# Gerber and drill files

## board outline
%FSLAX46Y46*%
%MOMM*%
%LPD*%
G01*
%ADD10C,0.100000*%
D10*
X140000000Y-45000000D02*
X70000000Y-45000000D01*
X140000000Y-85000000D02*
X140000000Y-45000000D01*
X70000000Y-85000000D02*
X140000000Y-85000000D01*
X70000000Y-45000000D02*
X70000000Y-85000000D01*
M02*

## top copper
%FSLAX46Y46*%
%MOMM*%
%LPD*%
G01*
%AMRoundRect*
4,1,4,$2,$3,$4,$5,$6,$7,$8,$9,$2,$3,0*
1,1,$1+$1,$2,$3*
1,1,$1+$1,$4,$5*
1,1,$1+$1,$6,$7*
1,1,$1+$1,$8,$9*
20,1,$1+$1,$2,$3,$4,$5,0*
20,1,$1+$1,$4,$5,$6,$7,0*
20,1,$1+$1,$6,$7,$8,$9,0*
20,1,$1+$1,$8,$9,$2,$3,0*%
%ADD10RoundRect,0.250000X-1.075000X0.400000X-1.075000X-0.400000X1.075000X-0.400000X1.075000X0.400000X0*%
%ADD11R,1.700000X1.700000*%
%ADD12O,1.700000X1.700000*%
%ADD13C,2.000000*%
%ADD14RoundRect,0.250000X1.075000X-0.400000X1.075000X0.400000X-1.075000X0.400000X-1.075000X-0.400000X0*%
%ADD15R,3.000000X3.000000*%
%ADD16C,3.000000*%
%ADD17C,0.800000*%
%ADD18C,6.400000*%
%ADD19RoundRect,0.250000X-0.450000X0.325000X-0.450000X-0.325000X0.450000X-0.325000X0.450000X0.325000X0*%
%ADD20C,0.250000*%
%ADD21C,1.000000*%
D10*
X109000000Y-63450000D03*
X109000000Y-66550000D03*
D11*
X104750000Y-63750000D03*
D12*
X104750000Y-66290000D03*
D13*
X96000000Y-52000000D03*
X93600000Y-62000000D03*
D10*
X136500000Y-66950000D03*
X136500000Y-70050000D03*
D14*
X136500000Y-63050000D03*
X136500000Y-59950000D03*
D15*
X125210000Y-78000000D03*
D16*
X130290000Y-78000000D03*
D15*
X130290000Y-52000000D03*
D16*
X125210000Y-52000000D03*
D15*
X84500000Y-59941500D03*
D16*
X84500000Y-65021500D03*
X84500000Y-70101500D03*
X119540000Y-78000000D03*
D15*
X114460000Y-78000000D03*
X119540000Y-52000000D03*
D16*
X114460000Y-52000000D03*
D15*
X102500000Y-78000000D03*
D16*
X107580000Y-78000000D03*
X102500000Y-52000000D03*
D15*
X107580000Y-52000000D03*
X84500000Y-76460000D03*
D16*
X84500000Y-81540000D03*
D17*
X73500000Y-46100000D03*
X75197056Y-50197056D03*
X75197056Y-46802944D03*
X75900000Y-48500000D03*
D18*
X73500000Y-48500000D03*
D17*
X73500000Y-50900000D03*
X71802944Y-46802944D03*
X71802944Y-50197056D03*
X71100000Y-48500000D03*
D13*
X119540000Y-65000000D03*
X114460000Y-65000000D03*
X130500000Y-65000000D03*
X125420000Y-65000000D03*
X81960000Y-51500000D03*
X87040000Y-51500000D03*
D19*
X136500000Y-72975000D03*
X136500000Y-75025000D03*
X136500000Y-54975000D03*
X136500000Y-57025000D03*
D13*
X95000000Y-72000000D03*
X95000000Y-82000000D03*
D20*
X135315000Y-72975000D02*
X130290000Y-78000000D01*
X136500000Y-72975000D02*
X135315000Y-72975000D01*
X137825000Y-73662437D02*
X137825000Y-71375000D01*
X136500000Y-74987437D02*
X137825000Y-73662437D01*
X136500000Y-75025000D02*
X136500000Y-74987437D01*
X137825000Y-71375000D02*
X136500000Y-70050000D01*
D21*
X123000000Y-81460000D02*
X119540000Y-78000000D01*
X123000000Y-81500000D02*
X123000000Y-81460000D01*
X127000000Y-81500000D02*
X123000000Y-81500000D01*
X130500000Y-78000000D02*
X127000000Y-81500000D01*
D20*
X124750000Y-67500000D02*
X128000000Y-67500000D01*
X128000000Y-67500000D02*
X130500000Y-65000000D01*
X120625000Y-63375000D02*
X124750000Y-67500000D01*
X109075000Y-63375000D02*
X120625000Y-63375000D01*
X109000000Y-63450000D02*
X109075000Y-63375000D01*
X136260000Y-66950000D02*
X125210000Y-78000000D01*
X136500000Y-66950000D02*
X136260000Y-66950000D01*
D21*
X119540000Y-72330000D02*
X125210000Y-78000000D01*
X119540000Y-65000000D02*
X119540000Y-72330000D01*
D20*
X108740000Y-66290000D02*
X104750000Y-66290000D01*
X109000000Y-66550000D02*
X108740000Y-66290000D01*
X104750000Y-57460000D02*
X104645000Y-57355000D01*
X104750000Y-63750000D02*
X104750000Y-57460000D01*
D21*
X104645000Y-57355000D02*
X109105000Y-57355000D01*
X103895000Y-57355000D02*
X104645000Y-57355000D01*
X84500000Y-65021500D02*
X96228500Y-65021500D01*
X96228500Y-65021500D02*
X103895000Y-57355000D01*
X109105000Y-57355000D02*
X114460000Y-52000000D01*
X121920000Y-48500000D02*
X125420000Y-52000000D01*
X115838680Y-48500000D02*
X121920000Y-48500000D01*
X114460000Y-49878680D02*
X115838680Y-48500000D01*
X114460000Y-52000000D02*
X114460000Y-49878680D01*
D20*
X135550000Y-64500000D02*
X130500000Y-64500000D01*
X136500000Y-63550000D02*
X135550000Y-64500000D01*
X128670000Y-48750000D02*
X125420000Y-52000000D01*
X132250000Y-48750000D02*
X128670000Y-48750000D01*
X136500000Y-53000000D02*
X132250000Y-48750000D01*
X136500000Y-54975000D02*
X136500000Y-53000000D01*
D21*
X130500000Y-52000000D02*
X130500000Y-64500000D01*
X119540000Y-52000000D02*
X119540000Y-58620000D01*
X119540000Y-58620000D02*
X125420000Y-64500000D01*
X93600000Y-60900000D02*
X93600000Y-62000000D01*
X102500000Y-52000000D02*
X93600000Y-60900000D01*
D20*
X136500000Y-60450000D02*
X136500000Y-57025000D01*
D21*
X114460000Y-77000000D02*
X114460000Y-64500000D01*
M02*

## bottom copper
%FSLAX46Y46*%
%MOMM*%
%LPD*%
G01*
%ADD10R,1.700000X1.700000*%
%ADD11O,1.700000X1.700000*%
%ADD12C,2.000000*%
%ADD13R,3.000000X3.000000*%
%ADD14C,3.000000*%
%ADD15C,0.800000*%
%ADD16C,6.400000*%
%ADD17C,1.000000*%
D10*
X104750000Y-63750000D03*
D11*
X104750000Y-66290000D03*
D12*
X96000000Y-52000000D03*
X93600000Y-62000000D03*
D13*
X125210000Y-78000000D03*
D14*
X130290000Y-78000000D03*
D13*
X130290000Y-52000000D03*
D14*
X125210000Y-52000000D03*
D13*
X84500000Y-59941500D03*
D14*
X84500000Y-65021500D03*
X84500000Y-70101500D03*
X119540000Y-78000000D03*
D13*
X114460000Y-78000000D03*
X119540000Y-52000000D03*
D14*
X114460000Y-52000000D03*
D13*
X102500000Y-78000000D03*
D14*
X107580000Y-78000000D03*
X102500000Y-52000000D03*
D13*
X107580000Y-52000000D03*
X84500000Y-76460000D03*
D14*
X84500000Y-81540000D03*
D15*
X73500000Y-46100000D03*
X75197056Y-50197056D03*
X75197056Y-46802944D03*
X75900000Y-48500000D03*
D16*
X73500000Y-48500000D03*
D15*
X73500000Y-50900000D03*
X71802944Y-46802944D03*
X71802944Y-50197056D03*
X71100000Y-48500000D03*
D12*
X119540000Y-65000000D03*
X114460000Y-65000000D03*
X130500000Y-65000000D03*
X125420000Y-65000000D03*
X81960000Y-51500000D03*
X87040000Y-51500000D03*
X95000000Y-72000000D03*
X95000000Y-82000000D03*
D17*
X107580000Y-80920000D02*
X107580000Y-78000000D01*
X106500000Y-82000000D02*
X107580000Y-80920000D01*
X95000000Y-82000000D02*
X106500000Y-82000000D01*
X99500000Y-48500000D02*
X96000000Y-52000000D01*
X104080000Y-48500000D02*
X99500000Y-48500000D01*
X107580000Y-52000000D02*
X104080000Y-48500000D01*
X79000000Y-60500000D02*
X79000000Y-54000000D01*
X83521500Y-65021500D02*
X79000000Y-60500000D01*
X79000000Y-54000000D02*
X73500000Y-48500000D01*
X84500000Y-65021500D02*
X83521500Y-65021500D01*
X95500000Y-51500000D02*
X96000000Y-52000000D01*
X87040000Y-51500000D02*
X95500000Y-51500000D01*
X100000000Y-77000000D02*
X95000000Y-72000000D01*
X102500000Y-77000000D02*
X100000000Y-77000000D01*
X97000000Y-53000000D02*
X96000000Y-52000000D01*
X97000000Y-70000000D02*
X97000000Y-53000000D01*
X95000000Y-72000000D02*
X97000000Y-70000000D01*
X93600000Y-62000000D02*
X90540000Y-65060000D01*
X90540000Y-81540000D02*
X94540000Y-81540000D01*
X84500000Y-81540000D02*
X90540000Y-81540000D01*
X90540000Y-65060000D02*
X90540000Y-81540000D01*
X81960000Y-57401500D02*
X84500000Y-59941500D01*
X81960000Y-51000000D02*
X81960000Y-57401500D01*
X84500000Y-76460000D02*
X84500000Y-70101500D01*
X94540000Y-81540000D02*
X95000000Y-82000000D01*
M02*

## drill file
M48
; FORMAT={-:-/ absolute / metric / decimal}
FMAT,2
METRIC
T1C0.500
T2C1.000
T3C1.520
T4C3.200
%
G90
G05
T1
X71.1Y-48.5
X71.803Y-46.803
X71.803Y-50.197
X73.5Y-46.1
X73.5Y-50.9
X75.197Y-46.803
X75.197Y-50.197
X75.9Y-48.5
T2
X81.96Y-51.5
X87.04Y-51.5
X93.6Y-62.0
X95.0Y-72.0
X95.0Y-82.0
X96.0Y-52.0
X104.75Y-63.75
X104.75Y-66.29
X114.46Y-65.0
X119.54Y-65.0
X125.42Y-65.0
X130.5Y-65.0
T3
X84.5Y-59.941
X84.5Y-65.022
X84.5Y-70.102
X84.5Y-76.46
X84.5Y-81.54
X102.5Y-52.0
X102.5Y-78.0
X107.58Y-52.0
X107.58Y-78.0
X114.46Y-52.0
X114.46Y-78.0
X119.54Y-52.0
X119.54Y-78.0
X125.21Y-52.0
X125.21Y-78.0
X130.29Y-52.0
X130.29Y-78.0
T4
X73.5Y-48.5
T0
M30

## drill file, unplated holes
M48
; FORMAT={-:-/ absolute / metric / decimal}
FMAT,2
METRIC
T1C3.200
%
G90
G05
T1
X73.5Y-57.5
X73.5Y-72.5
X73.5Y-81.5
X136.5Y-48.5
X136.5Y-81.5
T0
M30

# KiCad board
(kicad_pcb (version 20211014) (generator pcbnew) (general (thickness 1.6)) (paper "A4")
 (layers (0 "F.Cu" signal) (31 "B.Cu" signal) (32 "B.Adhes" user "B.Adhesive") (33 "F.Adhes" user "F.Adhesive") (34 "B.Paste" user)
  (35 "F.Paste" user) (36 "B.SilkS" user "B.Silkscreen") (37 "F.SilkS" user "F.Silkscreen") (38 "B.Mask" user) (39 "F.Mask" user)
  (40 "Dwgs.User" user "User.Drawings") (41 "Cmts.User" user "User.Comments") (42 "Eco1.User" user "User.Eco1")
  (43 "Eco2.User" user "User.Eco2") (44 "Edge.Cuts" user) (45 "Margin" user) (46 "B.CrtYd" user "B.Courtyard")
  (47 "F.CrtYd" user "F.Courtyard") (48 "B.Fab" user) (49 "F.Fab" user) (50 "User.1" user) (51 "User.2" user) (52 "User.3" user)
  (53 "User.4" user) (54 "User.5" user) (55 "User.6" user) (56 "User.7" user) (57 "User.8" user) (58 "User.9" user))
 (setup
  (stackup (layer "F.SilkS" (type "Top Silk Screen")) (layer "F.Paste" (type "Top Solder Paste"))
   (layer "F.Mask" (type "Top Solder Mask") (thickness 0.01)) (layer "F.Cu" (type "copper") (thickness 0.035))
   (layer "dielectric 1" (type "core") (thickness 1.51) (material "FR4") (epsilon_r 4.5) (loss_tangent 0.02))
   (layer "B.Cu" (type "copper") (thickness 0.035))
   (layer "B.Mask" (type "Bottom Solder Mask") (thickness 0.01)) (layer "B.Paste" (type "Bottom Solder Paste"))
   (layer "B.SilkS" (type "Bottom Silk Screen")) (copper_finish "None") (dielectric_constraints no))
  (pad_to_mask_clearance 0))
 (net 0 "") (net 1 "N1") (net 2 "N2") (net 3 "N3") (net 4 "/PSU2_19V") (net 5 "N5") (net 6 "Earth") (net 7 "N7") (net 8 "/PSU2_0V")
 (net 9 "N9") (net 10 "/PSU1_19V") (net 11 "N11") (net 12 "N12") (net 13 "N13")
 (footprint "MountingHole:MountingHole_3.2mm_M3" (layer "F.Cu") (at 73.5 57.5)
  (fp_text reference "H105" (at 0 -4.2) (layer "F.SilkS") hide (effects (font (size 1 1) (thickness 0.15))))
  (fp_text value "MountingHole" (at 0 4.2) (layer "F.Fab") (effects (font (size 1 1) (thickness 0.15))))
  (pad "" np_thru_hole circle (at 0 0) (size 3.2 3.2) (drill 3.2) (layers *.Cu *.Mask)))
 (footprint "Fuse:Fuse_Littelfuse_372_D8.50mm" (layer "F.Cu") (at 81.96 51.5)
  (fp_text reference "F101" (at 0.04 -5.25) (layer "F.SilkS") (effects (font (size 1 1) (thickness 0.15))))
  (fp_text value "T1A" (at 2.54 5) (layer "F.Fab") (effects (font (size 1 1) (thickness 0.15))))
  (pad "1" thru_hole circle (at 0 0) (size 2 2) (drill 1) (layers *.Cu *.Mask) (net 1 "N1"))
  (pad "2" thru_hole circle (at 5.08 0) (size 2 2) (drill 1) (layers *.Cu *.Mask) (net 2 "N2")))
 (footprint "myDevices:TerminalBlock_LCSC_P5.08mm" (layer "F.Cu") (at 102.5 78)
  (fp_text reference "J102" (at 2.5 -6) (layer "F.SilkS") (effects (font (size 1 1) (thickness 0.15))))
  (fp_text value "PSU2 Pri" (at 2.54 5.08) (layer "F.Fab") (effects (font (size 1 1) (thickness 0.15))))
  (pad "1" thru_hole rect locked (at 0 0) (size 3 3) (drill 1.52) (layers *.Cu *.Mask) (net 2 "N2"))
  (pad "2" thru_hole circle locked (at 5.08 0) (size 3 3) (drill 1.52) (layers *.Cu *.Mask) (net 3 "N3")))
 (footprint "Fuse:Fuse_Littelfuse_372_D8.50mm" (layer "F.Cu") (at 119.54 65 180)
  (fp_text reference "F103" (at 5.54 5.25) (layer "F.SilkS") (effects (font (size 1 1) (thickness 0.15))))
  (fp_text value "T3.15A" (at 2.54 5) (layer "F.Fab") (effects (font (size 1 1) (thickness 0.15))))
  (pad "1" thru_hole circle (at 0 0 180) (size 2 2) (drill 1) (layers *.Cu *.Mask) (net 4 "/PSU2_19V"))
  (pad "2" thru_hole circle (at 5.08 0 180) (size 2 2) (drill 1) (layers *.Cu *.Mask) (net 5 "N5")))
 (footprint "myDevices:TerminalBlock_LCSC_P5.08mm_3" (layer "F.Cu") (at 84.5 59.9415 -90)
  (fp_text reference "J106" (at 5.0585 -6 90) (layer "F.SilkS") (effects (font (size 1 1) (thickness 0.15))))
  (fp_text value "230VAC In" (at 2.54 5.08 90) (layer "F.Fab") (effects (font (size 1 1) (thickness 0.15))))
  (pad "1" thru_hole rect locked (at 0 0 270) (size 3 3) (drill 1.52) (layers *.Cu *.Mask) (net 1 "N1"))
  (pad "2" thru_hole circle locked (at 5.08 0 270) (size 3 3) (drill 1.52) (layers *.Cu *.Mask) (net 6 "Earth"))
  (pad "3" thru_hole circle locked (at 10.16 0 270) (size 3 3) (drill 1.52) (layers *.Cu *.Mask) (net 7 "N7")))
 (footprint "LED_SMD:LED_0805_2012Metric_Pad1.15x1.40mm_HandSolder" (layer "F.Cu") (at 136.5 74 -90)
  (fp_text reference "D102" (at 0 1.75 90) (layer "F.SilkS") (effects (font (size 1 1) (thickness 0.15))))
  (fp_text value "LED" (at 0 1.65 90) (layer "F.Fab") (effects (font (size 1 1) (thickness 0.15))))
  (pad "1" smd roundrect (at -1.025 0 270) (size 1.15 1.4) (layers "F.Cu" "F.Paste" "F.Mask") (roundrect_rratio 0.2173913043)
   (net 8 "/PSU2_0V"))
  (pad "2" smd roundrect (at 1.025 0 270) (size 1.15 1.4) (layers "F.Cu" "F.Paste" "F.Mask") (roundrect_rratio 0.2173913043) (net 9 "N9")))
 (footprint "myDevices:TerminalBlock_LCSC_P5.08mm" (layer "F.Cu") (at 130.29 52 180)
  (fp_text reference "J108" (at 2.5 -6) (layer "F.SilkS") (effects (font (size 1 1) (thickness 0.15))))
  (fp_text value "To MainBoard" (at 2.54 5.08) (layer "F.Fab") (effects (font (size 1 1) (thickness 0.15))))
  (pad "1" thru_hole rect locked (at 0 0 180) (size 3 3) (drill 1.52) (layers *.Cu *.Mask) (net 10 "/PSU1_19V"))
  (pad "2" thru_hole circle locked (at 5.08 0 180) (size 3 3) (drill 1.52) (layers *.Cu *.Mask) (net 6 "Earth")))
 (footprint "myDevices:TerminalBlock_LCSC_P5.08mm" (layer "F.Cu") (at 84.5 76.46 -90)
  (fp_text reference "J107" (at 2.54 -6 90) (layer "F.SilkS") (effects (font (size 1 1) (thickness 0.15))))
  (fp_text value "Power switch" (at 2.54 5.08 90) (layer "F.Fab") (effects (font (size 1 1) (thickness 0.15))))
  (pad "1" thru_hole rect locked (at 0 0 270) (size 3 3) (drill 1.52) (layers *.Cu *.Mask) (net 7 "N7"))
  (pad "2" thru_hole circle locked (at 5.08 0 270) (size 3 3) (drill 1.52) (layers *.Cu *.Mask) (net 3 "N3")))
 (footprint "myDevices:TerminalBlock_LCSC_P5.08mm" (layer "F.Cu") (at 119.54 52 180)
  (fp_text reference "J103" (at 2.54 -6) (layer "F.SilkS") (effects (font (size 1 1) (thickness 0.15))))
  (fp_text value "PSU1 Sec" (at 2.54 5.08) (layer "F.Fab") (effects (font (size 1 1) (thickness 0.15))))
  (pad "1" thru_hole rect locked (at 0 0 180) (size 3 3) (drill 1.52) (layers *.Cu *.Mask) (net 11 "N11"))
  (pad "2" thru_hole circle locked (at 5.08 0 180) (size 3 3) (drill 1.52) (layers *.Cu *.Mask) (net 6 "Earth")))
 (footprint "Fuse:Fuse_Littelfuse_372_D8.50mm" (layer "F.Cu") (at 130.5 65 180)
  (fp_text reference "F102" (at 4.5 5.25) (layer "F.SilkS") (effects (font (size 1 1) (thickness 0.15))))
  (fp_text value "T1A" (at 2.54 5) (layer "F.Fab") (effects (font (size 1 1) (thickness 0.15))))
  (pad "1" thru_hole circle (at 0 0 180) (size 2 2) (drill 1) (layers *.Cu *.Mask) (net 10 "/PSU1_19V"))
  (pad "2" thru_hole circle (at 5.08 0 180) (size 2 2) (drill 1) (layers *.Cu *.Mask) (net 11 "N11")))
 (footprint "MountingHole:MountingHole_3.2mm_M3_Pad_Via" (layer "F.Cu") (at 73.5 48.5)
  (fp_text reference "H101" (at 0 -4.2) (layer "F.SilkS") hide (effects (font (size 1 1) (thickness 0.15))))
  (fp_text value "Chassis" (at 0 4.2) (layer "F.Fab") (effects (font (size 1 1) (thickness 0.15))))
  (pad "1" thru_hole circle (at 0 2.4) (size 0.8 0.8) (drill 0.5) (layers *.Cu *.Mask) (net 6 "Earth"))
  (pad "1" thru_hole circle (at 0 0) (size 6.4 6.4) (drill 3.2) (layers *.Cu *.Mask) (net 6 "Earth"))
  (pad "1" thru_hole circle (at -1.697056 1.697056) (size 0.8 0.8) (drill 0.5) (layers *.Cu *.Mask) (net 6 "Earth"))
  (pad "1" thru_hole circle (at 0 -2.4) (size 0.8 0.8) (drill 0.5) (layers *.Cu *.Mask) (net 6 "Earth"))
  (pad "1" thru_hole circle (at 1.697056 1.697056) (size 0.8 0.8) (drill 0.5) (layers *.Cu *.Mask) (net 6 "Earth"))
  (pad "1" thru_hole circle (at 1.697056 -1.697056) (size 0.8 0.8) (drill 0.5) (layers *.Cu *.Mask) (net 6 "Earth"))
  (pad "1" thru_hole circle (at 2.4 0) (size 0.8 0.8) (drill 0.5) (layers *.Cu *.Mask) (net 6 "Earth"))
  (pad "1" thru_hole circle (at -1.697056 -1.697056) (size 0.8 0.8) (drill 0.5) (layers *.Cu *.Mask) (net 6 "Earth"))
  (pad "1" thru_hole circle (at -2.4 0) (size 0.8 0.8) (drill 0.5) (layers *.Cu *.Mask) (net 6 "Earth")))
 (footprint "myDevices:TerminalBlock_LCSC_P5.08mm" (layer "F.Cu") (at 125.21 78)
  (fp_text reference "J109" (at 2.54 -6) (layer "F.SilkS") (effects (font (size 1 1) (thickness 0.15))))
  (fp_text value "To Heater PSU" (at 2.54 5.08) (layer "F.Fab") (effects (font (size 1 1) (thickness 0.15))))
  (pad "1" thru_hole rect locked (at 0 0) (size 3 3) (drill 1.52) (layers *.Cu *.Mask) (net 4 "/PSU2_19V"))
  (pad "2" thru_hole circle locked (at 5.08 0) (size 3 3) (drill 1.52) (layers *.Cu *.Mask) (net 8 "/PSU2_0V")))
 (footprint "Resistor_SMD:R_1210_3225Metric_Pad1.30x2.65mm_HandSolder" (layer "F.Cu") (at 136.5 68.5 -90)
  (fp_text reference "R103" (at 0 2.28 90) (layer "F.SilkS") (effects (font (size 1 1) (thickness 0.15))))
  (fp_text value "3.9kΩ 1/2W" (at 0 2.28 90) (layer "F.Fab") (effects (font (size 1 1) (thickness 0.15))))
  (pad "1" smd roundrect (at -1.55 0 270) (size 1.3 2.65) (layers "F.Cu" "F.Paste" "F.Mask") (roundrect_rratio 0.1923076923)
   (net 4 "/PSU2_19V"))
  (pad "2" smd roundrect (at 1.55 0 270) (size 1.3 2.65) (layers "F.Cu" "F.Paste" "F.Mask") (roundrect_rratio 0.1923076923) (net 9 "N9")))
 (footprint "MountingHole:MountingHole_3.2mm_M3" (layer "F.Cu") (at 73.5 81.5)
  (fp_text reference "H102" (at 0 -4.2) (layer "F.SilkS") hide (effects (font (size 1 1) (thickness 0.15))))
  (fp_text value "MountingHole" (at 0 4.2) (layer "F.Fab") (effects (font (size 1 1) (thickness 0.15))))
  (pad "" np_thru_hole circle (at 0 0) (size 3.2 3.2) (drill 3.2) (layers *.Cu *.Mask)))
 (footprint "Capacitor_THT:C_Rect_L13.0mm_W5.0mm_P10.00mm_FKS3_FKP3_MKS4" (layer "F.Cu") (at 95 72 -90)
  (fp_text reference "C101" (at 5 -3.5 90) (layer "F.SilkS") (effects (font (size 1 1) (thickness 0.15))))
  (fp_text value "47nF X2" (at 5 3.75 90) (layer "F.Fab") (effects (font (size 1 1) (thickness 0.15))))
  (pad "1" thru_hole circle (at 0 0 270) (size 2 2) (drill 1) (layers *.Cu *.Mask) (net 2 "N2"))
  (pad "2" thru_hole circle (at 10 0 270) (size 2 2) (drill 1) (layers *.Cu *.Mask) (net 3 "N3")))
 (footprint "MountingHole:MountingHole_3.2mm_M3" (layer "F.Cu") (at 136.5 81.5)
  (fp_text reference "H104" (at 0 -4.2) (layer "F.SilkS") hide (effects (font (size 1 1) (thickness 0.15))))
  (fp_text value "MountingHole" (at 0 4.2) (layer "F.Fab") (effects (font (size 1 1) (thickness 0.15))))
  (pad "" np_thru_hole circle (at 0 0) (size 3.2 3.2) (drill 3.2) (layers *.Cu *.Mask)))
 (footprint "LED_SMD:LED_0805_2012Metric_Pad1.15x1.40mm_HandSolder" (layer "F.Cu") (at 136.5 56 -90)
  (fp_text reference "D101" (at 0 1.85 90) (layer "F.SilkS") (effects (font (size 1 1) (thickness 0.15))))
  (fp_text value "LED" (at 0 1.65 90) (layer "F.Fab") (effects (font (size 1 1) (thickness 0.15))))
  (pad "1" smd roundrect (at -1.025 0 270) (size 1.15 1.4) (layers "F.Cu" "F.Paste" "F.Mask") (roundrect_rratio 0.2173913043)
   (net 6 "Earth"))
  (pad "2" smd roundrect (at 1.025 0 270) (size 1.15 1.4) (layers "F.Cu" "F.Paste" "F.Mask") (roundrect_rratio 0.2173913043) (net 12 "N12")))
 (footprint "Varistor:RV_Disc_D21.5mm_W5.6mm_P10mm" (layer "F.Cu") (at 96 52 -90)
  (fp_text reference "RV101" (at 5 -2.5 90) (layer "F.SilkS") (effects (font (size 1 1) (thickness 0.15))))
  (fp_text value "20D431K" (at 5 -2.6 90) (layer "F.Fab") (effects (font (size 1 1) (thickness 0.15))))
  (pad "1" thru_hole circle (at 0 0 270) (size 2 2) (drill 1) (layers *.Cu *.Mask) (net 2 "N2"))
  (pad "2" thru_hole circle (at 10 2.4 270) (size 2 2) (drill 1) (layers *.Cu *.Mask) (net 3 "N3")))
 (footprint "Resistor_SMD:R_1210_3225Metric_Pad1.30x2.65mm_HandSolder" (layer "F.Cu") (at 136.5 61.5 90)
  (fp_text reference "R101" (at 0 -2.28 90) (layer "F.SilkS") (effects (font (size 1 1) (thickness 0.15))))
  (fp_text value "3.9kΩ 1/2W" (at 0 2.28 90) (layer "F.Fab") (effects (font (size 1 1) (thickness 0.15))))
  (pad "1" smd roundrect (at -1.55 0 90) (size 1.3 2.65) (layers "F.Cu" "F.Paste" "F.Mask") (roundrect_rratio 0.1923076923)
   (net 10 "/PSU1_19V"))
  (pad "2" smd roundrect (at 1.55 0 90) (size 1.3 2.65) (layers "F.Cu" "F.Paste" "F.Mask") (roundrect_rratio 0.1923076923) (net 12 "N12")))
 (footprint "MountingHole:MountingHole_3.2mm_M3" (layer "F.Cu") (at 136.5 48.5)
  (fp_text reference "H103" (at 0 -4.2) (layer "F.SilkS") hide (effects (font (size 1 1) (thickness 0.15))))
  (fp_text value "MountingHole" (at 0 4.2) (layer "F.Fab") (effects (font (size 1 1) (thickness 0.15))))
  (pad "" np_thru_hole circle (at 0 0) (size 3.2 3.2) (drill 3.2) (layers *.Cu *.Mask)))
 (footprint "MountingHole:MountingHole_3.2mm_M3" (layer "F.Cu") (at 73.5 72.5)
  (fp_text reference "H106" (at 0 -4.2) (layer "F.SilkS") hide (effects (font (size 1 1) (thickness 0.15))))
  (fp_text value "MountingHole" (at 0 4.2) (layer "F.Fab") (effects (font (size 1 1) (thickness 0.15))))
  (pad "" np_thru_hole circle (at 0 0) (size 3.2 3.2) (drill 3.2) (layers *.Cu *.Mask)))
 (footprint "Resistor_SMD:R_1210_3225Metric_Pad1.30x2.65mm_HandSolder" (layer "F.Cu") (at 109 65 -90)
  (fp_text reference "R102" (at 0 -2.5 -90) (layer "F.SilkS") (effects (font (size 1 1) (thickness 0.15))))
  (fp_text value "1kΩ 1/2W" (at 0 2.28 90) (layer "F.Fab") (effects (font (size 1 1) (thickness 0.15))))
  (pad "1" smd roundrect (at -1.55 0 270) (size 1.3 2.65) (layers "F.Cu" "F.Paste" "F.Mask") (roundrect_rratio 0.1923076923)
   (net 10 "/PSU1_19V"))
  (pad "2" smd roundrect (at 1.55 0 270) (size 1.3 2.65) (layers "F.Cu" "F.Paste" "F.Mask") (roundrect_rratio 0.1923076923) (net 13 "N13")))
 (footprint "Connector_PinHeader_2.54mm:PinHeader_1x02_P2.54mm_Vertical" (layer "F.Cu") (at 104.75 63.75)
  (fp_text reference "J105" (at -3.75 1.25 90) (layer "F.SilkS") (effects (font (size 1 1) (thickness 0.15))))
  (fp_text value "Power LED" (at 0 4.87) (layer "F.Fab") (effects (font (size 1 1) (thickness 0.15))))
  (pad "1" thru_hole rect (at 0 0) (size 1.7 1.7) (drill 1) (layers *.Cu *.Mask) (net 6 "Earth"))
  (pad "2" thru_hole oval (at 0 2.54) (size 1.7 1.7) (drill 1) (layers *.Cu *.Mask) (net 13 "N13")))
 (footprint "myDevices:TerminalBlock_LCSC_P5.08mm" (layer "F.Cu") (at 114.46 78)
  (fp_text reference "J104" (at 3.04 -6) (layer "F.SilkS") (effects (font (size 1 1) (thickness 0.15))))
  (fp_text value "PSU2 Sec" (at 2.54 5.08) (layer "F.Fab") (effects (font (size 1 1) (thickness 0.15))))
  (pad "1" thru_hole rect locked (at 0 0) (size 3 3) (drill 1.52) (layers *.Cu *.Mask) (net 5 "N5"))
  (pad "2" thru_hole circle locked (at 5.08 0) (size 3 3) (drill 1.52) (layers *.Cu *.Mask) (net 8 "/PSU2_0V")))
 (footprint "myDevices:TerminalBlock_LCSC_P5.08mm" (layer "F.Cu") (at 107.58 52 180)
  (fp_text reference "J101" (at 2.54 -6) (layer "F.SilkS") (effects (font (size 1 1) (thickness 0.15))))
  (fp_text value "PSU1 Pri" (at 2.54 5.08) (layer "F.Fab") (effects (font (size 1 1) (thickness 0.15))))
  (pad "1" thru_hole rect locked (at 0 0 180) (size 3 3) (drill 1.52) (layers *.Cu *.Mask) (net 2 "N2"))
  (pad "2" thru_hole circle locked (at 5.08 0 180) (size 3 3) (drill 1.52) (layers *.Cu *.Mask) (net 3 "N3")))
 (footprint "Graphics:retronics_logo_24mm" (layer "B.Cu") (at 122.497465 62.25 180)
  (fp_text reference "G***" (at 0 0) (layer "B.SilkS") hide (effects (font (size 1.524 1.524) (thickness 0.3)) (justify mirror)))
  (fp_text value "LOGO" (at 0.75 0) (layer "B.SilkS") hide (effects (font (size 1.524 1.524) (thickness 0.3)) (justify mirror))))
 (gr_line (start 140 85) (end 140 45) (layer "Edge.Cuts") (width 0.1))
 (gr_line (start 140 45) (end 70 45) (layer "Edge.Cuts") (width 0.1))
 (gr_line (start 70 45) (end 70 85) (layer "Edge.Cuts") (width 0.1))
 (gr_line (start 70 85) (end 140 85) (layer "Edge.Cuts") (width 0.1))
 (segment (start 97 70) (end 97 53) (width 1) (layer "B.Cu") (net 2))
 (segment (start 102.5 77) (end 100 77) (width 1) (layer "B.Cu") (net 2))
 (segment (start 97 53) (end 96 52) (width 1) (layer "B.Cu") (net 2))
 (segment (start 104.08 48.5) (end 99.5 48.5) (width 1) (layer "B.Cu") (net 2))
 (segment (start 87.04 51.5) (end 95.5 51.5) (width 1) (layer "B.Cu") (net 2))
 (segment (start 107.58 52) (end 104.08 48.5) (width 1) (layer "B.Cu") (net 2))
 (segment (start 99.5 48.5) (end 96 52) (width 1) (layer "B.Cu") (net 2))
 (segment (start 95.5 51.5) (end 96 52) (width 1) (layer "B.Cu") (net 2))
 (segment (start 100 77) (end 95 72) (width 1) (layer "B.Cu") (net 2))
 (segment (start 95 72) (end 97 70) (width 1) (layer "B.Cu") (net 2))
 (segment (start 93.6 60.9) (end 93.6 62) (width 1) (layer "F.Cu") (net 3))
 (segment (start 102.5 52) (end 93.6 60.9) (width 1) (layer "F.Cu") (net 3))
 (segment (start 107.58 80.92) (end 107.58 78) (width 1) (layer "B.Cu") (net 3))
 (segment (start 84.5 81.54) (end 90.54 81.54) (width 1) (layer "B.Cu") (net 3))
 (segment (start 106.5 82) (end 107.58 80.92) (width 1) (layer "B.Cu") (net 3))
 (segment (start 94.54 81.54) (end 95 82) (width 1) (layer "B.Cu") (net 3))
 (segment (start 95 82) (end 106.5 82) (width 1) (layer "B.Cu") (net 3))
 (segment (start 90.54 65.06) (end 90.54 81.54) (width 1) (layer "B.Cu") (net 3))
 (segment (start 90.54 81.54) (end 94.54 81.54) (width 1) (layer "B.Cu") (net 3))
 (segment (start 93.6 62) (end 90.54 65.06) (width 1) (layer "B.Cu") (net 3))
 (segment (start 109.105 57.355) (end 114.46 52) (width 1) (layer "F.Cu") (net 6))
 (segment (start 115.83868 48.5) (end 121.92 48.5) (width 1) (layer "F.Cu") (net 6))
 (segment (start 114.46 49.87868) (end 115.83868 48.5) (width 1) (layer "F.Cu") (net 6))
 (segment (start 114.46 52) (end 114.46 49.87868) (width 1) (layer "F.Cu") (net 6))
 (segment (start 136.5 54.975) (end 136.5 53) (width 0.25) (layer "F.Cu") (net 6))
 (segment (start 103.895 57.355) (end 104.645 57.355) (width 1) (layer "F.Cu") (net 6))
 (segment (start 96.2285 65.0215) (end 103.895 57.355) (width 1) (layer "F.Cu") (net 6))
 (segment (start 104.75 63.75) (end 104.75 57.46) (width 0.25) (layer "F.Cu") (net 6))
 (segment (start 132.25 48.75) (end 128.67 48.75) (width 0.25) (layer "F.Cu") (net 6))
 (segment (start 121.92 48.5) (end 125.42 52) (width 1) (layer "F.Cu") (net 6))
 (segment (start 136.5 53) (end 132.25 48.75) (width 0.25) (layer "F.Cu") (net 6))
 (segment (start 104.75 57.46) (end 104.645 57.355) (width 0.25) (layer "F.Cu") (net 6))
 (segment (start 104.645 57.355) (end 109.105 57.355) (width 1) (layer "F.Cu") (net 6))
 (segment (start 128.67 48.75) (end 125.42 52) (width 0.25) (layer "F.Cu") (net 6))
 (segment (start 84.5 65.0215) (end 96.2285 65.0215) (width 1) (layer "F.Cu") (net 6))
 (segment (start 84.5 65.0215) (end 83.5215 65.0215) (width 1) (layer "B.Cu") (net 6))
 (segment (start 83.5215 65.0215) (end 79 60.5) (width 1) (layer "B.Cu") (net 6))
 (segment (start 79 54) (end 73.5 48.5) (width 1) (layer "B.Cu") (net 6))
 (segment (start 79 60.5) (end 79 54) (width 1) (layer "B.Cu") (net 6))
 (segment (start 136.5 60.45) (end 136.5 57.025) (width 0.25) (layer "F.Cu") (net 12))
 (segment (start 130.5 78) (end 127 81.5) (width 1) (layer "F.Cu") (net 8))
 (segment (start 123 81.46) (end 119.54 78) (width 1) (layer "F.Cu") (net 8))
 (segment (start 135.315 72.975) (end 130.29 78) (width 0.25) (layer "F.Cu") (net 8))
 (segment (start 127 81.5) (end 123 81.5) (width 1) (layer "F.Cu") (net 8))
 (segment (start 123 81.5) (end 123 81.46) (width 1) (layer "F.Cu") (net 8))
 (segment (start 136.5 72.975) (end 135.315 72.975) (width 0.25) (layer "F.Cu") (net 8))
 (segment (start 136.5 75.025) (end 136.5 74.987437) (width 0.25) (layer "F.Cu") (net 9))
 (segment (start 137.825 73.662437) (end 137.825 71.375) (width 0.25) (layer "F.Cu") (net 9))
 (segment (start 136.5 74.987437) (end 137.825 73.662437) (width 0.25) (layer "F.Cu") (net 9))
 (segment (start 137.825 71.375) (end 136.5 70.05) (width 0.25) (layer "F.Cu") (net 9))
 (segment (start 81.96 51) (end 81.96 57.4015) (width 1) (layer "B.Cu") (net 1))
 (segment (start 81.96 57.4015) (end 84.5 59.9415) (width 1) (layer "B.Cu") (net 1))
 (segment (start 130.5 52) (end 130.5 64.5) (width 1) (layer "F.Cu") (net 10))
 (segment (start 136.5 63.55) (end 135.55 64.5) (width 0.25) (layer "F.Cu") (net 10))
 (segment (start 120.625 63.375) (end 124.75 67.5) (width 0.25) (layer "F.Cu") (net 10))
 (segment (start 128 67.5) (end 130.5 65) (width 0.25) (layer "F.Cu") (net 10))
 (segment (start 135.55 64.5) (end 130.5 64.5) (width 0.25) (layer "F.Cu") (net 10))
 (segment (start 124.75 67.5) (end 128 67.5) (width 0.25) (layer "F.Cu") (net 10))
 (segment (start 109 63.45) (end 109.075 63.375) (width 0.25) (layer "F.Cu") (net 10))
 (segment (start 109.075 63.375) (end 120.625 63.375) (width 0.25) (layer "F.Cu") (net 10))
 (segment (start 119.54 58.62) (end 125.42 64.5) (width 1) (layer "F.Cu") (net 11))
 (segment (start 119.54 52) (end 119.54 58.62) (width 1) (layer "F.Cu") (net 11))
 (segment (start 119.54 72.33) (end 125.21 78) (width 1) (layer "F.Cu") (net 4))
 (segment (start 136.5 66.95) (end 136.26 66.95) (width 0.25) (layer "F.Cu") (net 4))
 (segment (start 119.54 65) (end 119.54 72.33) (width 1) (layer "F.Cu") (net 4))
 (segment (start 136.26 66.95) (end 125.21 78) (width 0.25) (layer "F.Cu") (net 4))
 (segment (start 114.46 77) (end 114.46 64.5) (width 1) (layer "F.Cu") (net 5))
 (segment (start 84.5 76.46) (end 84.5 70.1015) (width 1) (layer "B.Cu") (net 7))
 (segment (start 108.74 66.29) (end 104.75 66.29) (width 0.25) (layer "F.Cu") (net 13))
 (segment (start 109 66.55) (end 108.74 66.29) (width 0.25) (layer "F.Cu") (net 13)))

